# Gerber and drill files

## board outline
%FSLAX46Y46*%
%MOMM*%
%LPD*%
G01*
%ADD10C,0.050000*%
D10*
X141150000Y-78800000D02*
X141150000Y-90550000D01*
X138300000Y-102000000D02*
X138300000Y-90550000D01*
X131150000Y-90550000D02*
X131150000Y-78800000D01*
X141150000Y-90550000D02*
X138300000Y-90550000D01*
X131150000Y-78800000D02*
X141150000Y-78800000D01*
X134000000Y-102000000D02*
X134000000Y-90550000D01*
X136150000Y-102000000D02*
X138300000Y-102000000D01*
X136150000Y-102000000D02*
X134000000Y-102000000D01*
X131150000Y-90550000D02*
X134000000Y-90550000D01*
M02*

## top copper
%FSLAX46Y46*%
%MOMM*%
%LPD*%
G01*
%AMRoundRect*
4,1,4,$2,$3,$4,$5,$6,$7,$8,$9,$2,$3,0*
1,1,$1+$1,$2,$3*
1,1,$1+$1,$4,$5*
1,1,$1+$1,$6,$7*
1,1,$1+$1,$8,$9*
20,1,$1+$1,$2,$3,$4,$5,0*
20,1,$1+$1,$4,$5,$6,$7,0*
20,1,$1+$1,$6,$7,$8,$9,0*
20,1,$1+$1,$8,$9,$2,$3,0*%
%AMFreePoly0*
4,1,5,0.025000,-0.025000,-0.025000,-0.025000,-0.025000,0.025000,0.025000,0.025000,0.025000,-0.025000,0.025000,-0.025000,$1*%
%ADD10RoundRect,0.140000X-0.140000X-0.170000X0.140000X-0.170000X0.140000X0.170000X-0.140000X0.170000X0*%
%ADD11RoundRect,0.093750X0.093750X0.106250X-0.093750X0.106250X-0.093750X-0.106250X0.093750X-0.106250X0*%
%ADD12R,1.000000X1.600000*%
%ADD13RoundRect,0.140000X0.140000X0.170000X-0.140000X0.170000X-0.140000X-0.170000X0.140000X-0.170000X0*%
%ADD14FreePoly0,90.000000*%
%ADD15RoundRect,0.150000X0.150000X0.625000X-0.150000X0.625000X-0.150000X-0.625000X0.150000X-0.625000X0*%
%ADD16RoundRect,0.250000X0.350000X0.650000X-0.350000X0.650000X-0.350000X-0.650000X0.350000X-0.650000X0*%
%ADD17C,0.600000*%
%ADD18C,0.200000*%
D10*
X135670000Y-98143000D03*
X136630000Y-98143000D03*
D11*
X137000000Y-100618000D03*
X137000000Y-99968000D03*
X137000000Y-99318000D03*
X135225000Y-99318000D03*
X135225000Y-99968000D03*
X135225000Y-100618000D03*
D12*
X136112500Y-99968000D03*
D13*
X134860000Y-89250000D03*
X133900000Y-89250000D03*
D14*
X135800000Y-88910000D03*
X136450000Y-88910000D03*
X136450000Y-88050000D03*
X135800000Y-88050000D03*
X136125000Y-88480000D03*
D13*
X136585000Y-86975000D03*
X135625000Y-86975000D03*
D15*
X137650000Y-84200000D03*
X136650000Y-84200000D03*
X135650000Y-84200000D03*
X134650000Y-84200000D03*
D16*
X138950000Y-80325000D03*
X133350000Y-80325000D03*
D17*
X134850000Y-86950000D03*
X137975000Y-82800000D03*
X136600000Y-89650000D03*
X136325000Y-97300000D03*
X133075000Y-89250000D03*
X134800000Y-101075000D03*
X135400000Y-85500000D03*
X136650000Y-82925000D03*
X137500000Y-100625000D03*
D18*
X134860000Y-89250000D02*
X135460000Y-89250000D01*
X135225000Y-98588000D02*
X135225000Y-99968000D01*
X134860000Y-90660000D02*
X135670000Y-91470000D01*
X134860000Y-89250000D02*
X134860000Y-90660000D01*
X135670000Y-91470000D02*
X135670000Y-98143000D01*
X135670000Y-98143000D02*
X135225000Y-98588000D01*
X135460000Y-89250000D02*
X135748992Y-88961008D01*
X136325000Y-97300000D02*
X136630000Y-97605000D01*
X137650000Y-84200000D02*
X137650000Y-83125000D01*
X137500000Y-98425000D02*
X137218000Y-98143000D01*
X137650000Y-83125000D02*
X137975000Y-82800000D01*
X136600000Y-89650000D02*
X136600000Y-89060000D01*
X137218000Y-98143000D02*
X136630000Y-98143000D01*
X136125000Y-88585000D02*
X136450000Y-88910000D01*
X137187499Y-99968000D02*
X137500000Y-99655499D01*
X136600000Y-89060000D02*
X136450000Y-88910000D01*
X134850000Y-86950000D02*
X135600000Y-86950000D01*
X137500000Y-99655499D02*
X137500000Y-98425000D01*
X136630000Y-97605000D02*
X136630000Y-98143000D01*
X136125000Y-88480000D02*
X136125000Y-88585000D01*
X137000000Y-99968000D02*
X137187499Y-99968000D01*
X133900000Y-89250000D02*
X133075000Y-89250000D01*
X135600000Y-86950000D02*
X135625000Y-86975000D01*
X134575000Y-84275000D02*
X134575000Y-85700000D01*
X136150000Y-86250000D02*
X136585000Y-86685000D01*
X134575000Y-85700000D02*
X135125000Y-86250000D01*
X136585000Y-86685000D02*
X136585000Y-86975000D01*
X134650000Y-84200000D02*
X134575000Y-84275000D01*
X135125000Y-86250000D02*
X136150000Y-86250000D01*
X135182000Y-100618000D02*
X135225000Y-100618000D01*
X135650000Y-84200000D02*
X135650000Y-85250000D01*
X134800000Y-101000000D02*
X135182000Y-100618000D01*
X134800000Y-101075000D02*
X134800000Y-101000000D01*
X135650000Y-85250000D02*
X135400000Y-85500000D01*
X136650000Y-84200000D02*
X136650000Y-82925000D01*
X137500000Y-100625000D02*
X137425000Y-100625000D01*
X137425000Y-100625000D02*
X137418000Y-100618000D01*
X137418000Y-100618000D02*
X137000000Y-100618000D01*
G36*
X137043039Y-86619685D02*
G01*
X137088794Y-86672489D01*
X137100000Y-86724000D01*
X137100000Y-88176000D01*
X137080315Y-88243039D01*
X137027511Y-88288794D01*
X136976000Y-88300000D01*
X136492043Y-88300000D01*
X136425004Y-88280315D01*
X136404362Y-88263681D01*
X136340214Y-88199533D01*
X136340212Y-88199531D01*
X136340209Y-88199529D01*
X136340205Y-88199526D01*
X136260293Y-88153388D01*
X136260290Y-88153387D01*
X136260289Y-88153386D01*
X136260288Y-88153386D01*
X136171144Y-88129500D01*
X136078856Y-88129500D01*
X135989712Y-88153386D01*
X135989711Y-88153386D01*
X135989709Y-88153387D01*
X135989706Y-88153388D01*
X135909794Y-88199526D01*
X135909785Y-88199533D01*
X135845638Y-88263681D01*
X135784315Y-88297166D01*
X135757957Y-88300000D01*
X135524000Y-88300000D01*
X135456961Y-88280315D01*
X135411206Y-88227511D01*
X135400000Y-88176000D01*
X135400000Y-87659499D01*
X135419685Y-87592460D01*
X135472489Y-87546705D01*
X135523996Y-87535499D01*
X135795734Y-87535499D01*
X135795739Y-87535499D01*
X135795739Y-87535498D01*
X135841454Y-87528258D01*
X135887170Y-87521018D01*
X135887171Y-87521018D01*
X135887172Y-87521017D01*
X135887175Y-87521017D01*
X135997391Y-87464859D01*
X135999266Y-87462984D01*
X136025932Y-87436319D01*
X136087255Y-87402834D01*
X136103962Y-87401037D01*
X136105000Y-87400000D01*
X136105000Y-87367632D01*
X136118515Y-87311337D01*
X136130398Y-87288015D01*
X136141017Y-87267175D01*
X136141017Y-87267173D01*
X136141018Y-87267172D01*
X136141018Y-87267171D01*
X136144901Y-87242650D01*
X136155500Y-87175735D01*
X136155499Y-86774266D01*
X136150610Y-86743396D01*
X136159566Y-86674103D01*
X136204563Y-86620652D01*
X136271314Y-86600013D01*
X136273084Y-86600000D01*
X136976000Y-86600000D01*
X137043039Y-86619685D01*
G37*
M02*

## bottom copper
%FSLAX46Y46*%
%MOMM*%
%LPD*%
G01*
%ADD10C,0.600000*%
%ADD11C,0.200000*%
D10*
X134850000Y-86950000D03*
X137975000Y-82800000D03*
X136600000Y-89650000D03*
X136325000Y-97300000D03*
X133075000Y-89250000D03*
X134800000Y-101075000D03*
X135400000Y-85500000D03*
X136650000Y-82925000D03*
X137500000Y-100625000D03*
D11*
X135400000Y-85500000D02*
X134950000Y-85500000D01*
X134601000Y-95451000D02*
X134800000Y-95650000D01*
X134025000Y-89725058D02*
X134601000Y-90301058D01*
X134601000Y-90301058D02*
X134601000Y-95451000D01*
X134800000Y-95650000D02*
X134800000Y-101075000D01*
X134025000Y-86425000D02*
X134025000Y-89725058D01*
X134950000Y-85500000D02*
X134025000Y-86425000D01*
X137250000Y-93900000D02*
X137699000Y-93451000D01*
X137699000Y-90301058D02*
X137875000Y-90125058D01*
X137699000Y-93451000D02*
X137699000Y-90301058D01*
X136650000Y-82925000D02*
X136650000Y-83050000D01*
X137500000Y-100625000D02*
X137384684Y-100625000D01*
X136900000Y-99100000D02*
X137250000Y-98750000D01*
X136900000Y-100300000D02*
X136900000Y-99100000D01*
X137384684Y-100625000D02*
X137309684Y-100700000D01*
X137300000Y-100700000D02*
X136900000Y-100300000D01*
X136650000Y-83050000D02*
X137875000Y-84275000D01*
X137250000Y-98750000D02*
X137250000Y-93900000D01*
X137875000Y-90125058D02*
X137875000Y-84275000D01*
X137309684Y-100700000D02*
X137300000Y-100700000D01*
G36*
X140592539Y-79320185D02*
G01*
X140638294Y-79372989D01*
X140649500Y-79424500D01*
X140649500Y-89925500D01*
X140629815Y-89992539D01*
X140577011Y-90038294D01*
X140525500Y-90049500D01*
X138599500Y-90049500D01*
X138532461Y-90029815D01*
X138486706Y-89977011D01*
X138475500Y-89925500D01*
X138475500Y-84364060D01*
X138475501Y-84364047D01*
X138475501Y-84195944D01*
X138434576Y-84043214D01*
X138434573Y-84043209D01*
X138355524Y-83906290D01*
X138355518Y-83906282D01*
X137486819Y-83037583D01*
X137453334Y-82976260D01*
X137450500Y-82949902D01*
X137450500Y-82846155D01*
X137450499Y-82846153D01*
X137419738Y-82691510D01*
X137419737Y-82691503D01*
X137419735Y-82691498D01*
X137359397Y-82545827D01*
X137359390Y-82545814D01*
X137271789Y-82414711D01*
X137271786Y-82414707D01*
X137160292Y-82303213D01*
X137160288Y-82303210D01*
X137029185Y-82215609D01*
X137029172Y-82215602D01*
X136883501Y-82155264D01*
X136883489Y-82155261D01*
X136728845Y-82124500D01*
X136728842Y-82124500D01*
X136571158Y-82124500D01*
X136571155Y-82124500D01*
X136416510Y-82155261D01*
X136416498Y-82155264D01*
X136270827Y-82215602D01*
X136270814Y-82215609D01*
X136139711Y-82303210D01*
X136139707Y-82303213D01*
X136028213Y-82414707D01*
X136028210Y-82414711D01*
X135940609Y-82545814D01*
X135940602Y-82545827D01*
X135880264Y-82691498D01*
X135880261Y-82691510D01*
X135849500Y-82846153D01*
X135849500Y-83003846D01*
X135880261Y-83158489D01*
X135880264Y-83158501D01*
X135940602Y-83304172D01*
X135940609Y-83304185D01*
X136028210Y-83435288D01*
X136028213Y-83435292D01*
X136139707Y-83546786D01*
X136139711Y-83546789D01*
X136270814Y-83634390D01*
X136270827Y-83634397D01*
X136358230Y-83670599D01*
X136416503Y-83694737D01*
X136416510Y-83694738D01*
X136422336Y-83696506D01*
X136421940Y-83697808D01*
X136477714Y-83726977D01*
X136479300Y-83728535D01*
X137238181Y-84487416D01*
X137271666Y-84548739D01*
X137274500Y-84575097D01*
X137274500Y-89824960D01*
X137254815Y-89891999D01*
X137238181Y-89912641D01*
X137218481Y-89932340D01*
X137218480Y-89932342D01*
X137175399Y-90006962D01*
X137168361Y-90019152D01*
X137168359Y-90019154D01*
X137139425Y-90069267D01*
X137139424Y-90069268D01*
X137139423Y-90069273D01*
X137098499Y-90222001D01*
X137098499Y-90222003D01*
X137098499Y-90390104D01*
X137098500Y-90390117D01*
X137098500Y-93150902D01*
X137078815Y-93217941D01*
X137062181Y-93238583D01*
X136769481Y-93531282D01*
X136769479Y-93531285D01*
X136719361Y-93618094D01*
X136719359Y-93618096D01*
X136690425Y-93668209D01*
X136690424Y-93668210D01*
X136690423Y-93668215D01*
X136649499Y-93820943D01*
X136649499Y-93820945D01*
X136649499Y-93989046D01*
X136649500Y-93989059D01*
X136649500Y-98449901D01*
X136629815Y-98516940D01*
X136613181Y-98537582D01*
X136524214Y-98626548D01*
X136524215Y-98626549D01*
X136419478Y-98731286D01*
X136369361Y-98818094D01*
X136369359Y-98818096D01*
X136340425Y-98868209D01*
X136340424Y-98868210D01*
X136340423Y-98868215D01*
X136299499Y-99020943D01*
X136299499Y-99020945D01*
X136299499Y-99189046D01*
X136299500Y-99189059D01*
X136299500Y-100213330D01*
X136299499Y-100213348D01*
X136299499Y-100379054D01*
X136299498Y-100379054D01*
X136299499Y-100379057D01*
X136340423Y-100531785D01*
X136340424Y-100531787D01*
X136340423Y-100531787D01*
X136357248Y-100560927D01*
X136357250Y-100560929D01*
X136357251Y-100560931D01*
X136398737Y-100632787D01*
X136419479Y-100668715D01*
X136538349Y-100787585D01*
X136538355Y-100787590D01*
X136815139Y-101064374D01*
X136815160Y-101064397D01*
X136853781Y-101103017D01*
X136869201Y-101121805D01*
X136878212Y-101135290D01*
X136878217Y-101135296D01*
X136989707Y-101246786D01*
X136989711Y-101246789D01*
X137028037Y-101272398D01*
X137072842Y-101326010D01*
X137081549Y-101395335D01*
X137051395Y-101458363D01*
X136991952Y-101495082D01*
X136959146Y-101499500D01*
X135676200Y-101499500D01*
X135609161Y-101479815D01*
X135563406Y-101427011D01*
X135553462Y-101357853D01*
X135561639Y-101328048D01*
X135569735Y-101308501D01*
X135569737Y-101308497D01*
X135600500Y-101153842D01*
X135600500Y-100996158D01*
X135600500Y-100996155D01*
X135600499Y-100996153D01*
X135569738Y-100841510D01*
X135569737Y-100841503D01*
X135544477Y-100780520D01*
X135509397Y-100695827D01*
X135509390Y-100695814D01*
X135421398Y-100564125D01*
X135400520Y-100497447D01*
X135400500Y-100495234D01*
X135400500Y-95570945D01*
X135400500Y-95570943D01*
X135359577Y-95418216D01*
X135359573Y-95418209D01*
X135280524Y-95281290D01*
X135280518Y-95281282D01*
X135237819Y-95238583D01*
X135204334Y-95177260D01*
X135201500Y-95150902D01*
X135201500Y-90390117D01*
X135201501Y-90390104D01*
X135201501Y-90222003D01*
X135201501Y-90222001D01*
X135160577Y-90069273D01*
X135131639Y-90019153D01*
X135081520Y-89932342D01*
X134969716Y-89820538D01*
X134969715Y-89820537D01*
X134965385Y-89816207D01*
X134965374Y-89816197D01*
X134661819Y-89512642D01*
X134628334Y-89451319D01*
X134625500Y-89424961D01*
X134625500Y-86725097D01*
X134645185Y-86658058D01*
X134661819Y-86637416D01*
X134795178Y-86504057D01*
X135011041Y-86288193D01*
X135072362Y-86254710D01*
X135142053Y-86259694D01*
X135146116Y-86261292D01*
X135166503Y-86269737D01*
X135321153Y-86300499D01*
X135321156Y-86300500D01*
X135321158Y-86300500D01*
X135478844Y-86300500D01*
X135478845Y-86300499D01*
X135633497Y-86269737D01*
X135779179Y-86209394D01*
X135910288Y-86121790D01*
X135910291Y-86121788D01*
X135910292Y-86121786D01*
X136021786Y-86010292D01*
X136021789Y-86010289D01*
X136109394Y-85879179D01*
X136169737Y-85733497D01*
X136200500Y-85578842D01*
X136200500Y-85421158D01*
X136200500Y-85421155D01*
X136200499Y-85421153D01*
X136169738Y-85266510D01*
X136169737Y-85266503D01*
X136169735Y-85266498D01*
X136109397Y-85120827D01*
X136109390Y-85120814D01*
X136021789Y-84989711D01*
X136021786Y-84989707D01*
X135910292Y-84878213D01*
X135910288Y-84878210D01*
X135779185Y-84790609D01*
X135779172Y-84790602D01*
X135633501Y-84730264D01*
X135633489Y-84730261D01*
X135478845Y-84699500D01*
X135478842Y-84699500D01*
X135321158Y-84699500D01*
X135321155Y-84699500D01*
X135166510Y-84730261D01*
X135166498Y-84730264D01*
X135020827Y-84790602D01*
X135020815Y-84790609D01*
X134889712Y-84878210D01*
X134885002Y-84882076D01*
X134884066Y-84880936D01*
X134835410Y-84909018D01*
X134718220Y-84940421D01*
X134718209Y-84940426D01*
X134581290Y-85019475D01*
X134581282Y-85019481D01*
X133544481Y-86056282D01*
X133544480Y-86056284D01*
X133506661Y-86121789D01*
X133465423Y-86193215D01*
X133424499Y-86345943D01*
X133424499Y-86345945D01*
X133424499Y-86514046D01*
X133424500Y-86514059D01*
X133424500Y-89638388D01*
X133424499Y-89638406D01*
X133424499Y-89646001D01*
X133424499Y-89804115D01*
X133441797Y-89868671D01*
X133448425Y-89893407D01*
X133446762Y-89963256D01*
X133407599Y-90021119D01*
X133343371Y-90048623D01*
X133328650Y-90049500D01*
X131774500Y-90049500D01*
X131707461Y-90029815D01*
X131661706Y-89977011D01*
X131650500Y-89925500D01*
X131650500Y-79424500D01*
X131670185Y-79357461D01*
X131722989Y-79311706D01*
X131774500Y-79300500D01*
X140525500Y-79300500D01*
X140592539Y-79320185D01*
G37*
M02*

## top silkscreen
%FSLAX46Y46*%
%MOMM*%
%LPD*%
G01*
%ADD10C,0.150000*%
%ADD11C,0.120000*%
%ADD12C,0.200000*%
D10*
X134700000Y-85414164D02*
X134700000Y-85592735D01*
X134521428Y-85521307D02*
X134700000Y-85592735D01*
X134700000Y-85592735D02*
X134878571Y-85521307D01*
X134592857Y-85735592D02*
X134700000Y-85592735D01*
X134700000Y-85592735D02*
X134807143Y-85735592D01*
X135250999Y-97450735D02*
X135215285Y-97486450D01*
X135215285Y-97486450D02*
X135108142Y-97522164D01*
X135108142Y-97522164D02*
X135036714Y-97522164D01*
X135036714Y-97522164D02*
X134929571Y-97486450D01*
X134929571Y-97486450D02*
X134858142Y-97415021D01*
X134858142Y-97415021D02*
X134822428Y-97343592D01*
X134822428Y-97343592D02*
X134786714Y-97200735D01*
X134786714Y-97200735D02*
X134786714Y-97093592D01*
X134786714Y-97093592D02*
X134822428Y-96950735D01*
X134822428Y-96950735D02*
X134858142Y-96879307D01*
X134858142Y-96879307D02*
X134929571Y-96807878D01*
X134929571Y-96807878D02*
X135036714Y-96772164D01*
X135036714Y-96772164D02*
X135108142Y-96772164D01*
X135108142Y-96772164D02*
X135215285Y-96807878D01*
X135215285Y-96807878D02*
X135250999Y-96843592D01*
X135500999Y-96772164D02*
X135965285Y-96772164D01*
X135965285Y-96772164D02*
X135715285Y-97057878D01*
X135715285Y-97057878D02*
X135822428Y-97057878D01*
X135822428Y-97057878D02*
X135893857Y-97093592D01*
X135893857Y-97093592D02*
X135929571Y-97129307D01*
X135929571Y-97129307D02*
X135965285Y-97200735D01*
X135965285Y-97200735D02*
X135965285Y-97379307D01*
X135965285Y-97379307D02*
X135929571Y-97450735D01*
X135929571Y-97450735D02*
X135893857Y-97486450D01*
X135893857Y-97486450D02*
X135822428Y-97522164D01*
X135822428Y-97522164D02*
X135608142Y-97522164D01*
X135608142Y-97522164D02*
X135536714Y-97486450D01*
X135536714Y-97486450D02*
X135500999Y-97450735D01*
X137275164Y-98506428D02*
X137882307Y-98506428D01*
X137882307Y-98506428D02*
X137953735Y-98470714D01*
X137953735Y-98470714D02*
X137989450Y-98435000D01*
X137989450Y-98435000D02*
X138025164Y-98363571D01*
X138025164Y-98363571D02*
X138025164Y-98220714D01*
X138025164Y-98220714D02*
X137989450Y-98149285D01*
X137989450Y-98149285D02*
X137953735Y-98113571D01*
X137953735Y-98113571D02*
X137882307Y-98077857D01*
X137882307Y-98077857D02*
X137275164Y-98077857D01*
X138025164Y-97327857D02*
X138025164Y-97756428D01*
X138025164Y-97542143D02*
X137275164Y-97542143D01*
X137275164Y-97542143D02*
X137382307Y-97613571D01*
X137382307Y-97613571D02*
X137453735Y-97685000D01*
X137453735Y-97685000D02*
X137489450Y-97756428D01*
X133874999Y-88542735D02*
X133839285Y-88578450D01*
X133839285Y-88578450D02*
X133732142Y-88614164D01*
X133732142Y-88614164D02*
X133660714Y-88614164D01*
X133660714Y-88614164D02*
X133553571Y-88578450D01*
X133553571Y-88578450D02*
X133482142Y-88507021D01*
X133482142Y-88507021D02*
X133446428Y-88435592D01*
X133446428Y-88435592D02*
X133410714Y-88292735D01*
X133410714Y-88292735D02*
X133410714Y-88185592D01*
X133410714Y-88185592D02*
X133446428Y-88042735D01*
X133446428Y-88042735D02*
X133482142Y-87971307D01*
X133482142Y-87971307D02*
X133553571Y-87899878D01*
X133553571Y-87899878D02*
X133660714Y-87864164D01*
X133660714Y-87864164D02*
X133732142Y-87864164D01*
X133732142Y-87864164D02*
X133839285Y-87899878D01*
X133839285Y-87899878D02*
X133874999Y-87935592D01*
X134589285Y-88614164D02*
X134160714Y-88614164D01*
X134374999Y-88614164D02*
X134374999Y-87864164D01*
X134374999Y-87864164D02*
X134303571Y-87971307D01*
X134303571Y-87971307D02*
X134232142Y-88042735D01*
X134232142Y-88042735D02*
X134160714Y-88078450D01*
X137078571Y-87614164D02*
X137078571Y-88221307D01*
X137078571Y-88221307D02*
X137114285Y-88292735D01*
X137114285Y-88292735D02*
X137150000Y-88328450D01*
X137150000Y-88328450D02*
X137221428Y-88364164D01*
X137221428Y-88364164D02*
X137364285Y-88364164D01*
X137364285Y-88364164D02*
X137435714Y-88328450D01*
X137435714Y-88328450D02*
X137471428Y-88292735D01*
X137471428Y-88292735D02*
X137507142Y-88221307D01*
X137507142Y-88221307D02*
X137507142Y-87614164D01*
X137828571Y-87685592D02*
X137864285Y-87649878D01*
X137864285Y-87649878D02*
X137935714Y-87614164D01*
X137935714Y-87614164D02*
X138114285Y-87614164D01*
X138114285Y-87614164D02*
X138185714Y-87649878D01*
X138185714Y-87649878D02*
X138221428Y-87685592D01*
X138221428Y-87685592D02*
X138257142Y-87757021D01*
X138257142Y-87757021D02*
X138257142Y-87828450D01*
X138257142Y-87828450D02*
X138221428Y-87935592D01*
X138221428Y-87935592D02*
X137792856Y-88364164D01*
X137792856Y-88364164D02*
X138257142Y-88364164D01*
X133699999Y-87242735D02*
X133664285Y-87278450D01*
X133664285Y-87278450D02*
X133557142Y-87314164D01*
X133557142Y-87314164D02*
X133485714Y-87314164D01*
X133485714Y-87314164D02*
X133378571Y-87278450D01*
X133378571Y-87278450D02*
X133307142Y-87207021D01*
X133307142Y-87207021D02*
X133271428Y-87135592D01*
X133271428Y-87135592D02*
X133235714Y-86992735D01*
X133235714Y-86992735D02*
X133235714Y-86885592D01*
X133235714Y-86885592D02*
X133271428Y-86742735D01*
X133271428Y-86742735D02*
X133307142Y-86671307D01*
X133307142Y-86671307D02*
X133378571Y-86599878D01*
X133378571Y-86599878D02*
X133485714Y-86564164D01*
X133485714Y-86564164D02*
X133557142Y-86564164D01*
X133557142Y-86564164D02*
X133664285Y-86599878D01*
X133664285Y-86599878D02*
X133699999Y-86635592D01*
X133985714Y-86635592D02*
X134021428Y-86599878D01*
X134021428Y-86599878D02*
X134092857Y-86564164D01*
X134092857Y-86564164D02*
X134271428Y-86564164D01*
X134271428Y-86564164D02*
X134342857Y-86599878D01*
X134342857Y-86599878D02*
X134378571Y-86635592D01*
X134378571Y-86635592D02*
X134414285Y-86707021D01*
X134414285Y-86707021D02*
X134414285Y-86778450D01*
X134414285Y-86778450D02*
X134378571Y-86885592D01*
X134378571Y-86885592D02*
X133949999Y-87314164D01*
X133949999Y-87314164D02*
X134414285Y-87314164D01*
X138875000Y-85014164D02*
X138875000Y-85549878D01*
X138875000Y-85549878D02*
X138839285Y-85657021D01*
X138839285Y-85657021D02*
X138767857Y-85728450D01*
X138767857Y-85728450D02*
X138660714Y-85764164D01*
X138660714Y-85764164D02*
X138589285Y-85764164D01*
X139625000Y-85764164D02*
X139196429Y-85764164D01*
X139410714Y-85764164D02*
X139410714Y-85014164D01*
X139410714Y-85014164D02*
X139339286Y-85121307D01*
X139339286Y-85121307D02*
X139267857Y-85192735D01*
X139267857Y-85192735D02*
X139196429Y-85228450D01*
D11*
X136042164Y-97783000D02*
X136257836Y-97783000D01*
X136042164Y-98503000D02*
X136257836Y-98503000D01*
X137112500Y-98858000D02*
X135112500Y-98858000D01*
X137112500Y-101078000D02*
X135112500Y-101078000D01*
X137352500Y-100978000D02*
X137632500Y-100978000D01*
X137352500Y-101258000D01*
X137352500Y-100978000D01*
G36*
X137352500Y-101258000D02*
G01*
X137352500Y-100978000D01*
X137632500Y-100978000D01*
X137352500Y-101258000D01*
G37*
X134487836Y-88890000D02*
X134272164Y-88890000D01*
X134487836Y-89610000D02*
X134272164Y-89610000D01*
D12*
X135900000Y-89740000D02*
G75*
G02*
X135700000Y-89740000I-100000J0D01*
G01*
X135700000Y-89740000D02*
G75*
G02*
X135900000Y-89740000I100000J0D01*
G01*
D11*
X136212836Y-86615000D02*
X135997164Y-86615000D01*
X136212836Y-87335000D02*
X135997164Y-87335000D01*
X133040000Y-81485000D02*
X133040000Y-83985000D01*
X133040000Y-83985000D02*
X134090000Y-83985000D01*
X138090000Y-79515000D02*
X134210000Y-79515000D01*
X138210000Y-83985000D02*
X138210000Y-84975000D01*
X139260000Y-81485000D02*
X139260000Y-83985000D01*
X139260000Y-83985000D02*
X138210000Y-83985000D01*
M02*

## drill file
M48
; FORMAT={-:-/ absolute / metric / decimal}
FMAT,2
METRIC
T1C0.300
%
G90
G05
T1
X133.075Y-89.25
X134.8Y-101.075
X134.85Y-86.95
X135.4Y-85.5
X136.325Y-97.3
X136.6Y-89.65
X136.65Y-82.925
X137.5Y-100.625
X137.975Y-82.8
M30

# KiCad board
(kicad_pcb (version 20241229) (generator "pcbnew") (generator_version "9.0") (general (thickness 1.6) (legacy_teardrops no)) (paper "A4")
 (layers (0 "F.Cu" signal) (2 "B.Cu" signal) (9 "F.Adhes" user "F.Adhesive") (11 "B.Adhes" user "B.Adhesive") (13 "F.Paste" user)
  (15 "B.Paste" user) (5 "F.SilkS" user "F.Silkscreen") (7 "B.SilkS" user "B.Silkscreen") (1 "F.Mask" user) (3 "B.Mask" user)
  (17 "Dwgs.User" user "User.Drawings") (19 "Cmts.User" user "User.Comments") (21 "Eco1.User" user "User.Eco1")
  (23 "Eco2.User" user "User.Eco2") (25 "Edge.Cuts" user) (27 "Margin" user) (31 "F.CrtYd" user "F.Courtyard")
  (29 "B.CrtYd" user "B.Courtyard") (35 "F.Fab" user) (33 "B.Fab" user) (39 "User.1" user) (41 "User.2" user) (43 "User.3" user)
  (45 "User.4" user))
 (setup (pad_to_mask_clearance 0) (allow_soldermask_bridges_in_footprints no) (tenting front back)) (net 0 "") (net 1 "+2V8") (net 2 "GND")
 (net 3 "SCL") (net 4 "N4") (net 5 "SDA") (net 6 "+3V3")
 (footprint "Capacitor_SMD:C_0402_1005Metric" (layer "F.Cu") (at 136.15 98.143)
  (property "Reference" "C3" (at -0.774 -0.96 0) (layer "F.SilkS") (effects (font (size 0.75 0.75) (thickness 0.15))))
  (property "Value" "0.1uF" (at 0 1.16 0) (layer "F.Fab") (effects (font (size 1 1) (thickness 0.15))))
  (fp_line (start -0.107836 -0.36) (end 0.107836 -0.36) (stroke (width 0.12) (type solid)) (layer "F.SilkS"))
  (fp_line (start -0.107836 0.36) (end 0.107836 0.36) (stroke (width 0.12) (type solid)) (layer "F.SilkS"))
  (pad "1" smd roundrect (at -0.48 0) (size 0.56 0.62) (layers "F.Cu" "F.Mask" "F.Paste") (roundrect_rratio 0.25) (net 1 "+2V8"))
  (pad "2" smd roundrect (at 0.48 0) (size 0.56 0.62) (layers "F.Cu" "F.Mask" "F.Paste") (roundrect_rratio 0.25) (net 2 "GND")))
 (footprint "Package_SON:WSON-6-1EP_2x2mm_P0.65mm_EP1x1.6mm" (layer "F.Cu") (at 136.1125 99.968 180)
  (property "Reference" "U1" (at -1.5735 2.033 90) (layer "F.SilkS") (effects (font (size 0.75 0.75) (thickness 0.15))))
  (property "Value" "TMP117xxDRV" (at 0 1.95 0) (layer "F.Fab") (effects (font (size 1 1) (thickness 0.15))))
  (fp_line (start -1 1.11) (end 1 1.11) (stroke (width 0.12) (type solid)) (layer "F.SilkS"))
  (fp_line (start -1 -1.11) (end 1 -1.11) (stroke (width 0.12) (type solid)) (layer "F.SilkS"))
  (fp_poly (pts (xy -1.24 -1.01) (xy -1.52 -1.01) (xy -1.24 -1.29)) (stroke (width 0.12) (type solid)) (fill yes) (layer "F.SilkS"))
  (pad "" smd roundrect (at 0 -0.4 180) (size 0.81 0.64) (layers "F.Paste") (roundrect_rratio 0.25))
  (pad "" smd roundrect (at 0 0.4 180) (size 0.81 0.64) (layers "F.Paste") (roundrect_rratio 0.25))
  (pad "1" smd roundrect (at -0.8875 -0.65 180) (size 0.375 0.4) (layers "F.Cu" "F.Mask" "F.Paste") (roundrect_rratio 0.25) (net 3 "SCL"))
  (pad "2" smd roundrect (at -0.8875 0 180) (size 0.375 0.4) (layers "F.Cu" "F.Mask" "F.Paste") (roundrect_rratio 0.25) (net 2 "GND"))
  (pad "3" smd roundrect (at -0.8875 0.65 180) (size 0.375 0.4) (layers "F.Cu" "F.Mask" "F.Paste") (roundrect_rratio 0.25) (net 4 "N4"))
  (pad "4" smd roundrect (at 0.8875 0.65 180) (size 0.375 0.4) (layers "F.Cu" "F.Mask" "F.Paste") (roundrect_rratio 0.25) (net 1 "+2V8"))
  (pad "5" smd roundrect (at 0.8875 0 180) (size 0.375 0.4) (layers "F.Cu" "F.Mask" "F.Paste") (roundrect_rratio 0.25) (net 1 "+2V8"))
  (pad "6" smd roundrect (at 0.8875 -0.65 180) (size 0.375 0.4) (layers "F.Cu" "F.Mask" "F.Paste") (roundrect_rratio 0.25) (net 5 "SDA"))
  (pad "7" smd rect (at 0 0 180) (size 1 1.6) (layers "F.Cu" "F.Mask") (zone_connect 2)))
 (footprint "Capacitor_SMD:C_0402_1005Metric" (layer "F.Cu") (at 134.38 89.25 180)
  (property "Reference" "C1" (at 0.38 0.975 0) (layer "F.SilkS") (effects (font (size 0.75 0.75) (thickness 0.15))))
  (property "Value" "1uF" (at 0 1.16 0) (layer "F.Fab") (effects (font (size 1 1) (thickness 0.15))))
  (fp_line (start -0.107836 0.36) (end 0.107836 0.36) (stroke (width 0.12) (type solid)) (layer "F.SilkS"))
  (fp_line (start -0.107836 -0.36) (end 0.107836 -0.36) (stroke (width 0.12) (type solid)) (layer "F.SilkS"))
  (pad "1" smd roundrect (at -0.48 0 180) (size 0.56 0.62) (layers "F.Cu" "F.Mask" "F.Paste") (roundrect_rratio 0.25) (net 1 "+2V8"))
  (pad "2" smd roundrect (at 0.48 0 180) (size 0.56 0.62) (layers "F.Cu" "F.Mask" "F.Paste") (roundrect_rratio 0.25) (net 2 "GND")))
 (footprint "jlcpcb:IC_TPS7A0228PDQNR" (layer "F.Cu") (at 136.125 88.48 90)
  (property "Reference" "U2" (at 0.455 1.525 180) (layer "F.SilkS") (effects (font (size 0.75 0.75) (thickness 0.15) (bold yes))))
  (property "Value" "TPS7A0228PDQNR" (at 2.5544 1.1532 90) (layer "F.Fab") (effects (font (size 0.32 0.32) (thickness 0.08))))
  (fp_circle (center -1.26 -0.325) (end -1.16 -0.325) (stroke (width 0.2) (type solid)) (fill no) (layer "F.SilkS"))
  (pad "1" smd custom (at -0.43 -0.325 90) (size 0.05 0.05) (layers "F.Cu") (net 1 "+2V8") (options (clearance outline) (anchor rect))
   (primitives))
  (pad "2" smd custom (at -0.43 0.325 90) (size 0.05 0.05) (layers "F.Cu") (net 2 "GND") (options (clearance outline) (anchor rect))
   (primitives))
  (pad "3" smd custom (at 0.43 0.325 90) (size 0.05 0.05) (layers "F.Cu") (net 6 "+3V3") (options (clearance outline) (anchor rect))
   (primitives))
  (pad "4" smd custom (at 0.43 -0.325 90) (size 0.05 0.05) (layers "F.Cu") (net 6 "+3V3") (options (clearance outline) (anchor rect))
   (primitives))
  (pad "5" smd custom (at 0 0 90) (size 0.05 0.05) (layers "F.Cu") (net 2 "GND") (options (clearance outline) (anchor rect)) (primitives)))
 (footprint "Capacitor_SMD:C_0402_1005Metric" (layer "F.Cu") (at 136.105 86.975 180)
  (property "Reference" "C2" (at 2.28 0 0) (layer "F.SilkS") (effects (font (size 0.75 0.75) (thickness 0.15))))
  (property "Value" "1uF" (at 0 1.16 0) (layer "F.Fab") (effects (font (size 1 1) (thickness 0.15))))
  (fp_line (start -0.107836 0.36) (end 0.107836 0.36) (stroke (width 0.12) (type solid)) (layer "F.SilkS"))
  (fp_line (start -0.107836 -0.36) (end 0.107836 -0.36) (stroke (width 0.12) (type solid)) (layer "F.SilkS"))
  (pad "1" smd roundrect (at -0.48 0 180) (size 0.56 0.62) (layers "F.Cu" "F.Mask" "F.Paste") (roundrect_rratio 0.25) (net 6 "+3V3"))
  (pad "2" smd roundrect (at 0.48 0 180) (size 0.56 0.62) (layers "F.Cu" "F.Mask" "F.Paste") (roundrect_rratio 0.25) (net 2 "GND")))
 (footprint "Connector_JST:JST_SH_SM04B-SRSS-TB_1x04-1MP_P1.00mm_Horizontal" (layer "F.Cu") (at 136.15 82.2 180)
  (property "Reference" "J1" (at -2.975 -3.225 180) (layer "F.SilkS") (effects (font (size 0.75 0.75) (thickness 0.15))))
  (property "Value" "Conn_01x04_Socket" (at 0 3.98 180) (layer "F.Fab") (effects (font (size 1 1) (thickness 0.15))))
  (fp_line (start 3.11 0.715) (end 3.11 -1.785) (stroke (width 0.12) (type solid)) (layer "F.SilkS"))
  (fp_line (start 3.11 -1.785) (end 2.06 -1.785) (stroke (width 0.12) (type solid)) (layer "F.SilkS"))
  (fp_line (start -1.94 2.685) (end 1.94 2.685) (stroke (width 0.12) (type solid)) (layer "F.SilkS"))
  (fp_line (start -2.06 -1.785) (end -2.06 -2.775) (stroke (width 0.12) (type solid)) (layer "F.SilkS"))
  (fp_line (start -3.11 0.715) (end -3.11 -1.785) (stroke (width 0.12) (type solid)) (layer "F.SilkS"))
  (fp_line (start -3.11 -1.785) (end -2.06 -1.785) (stroke (width 0.12) (type solid)) (layer "F.SilkS"))
  (pad "1" smd roundrect (at -1.5 -2 180) (size 0.6 1.55) (layers "F.Cu" "F.Mask" "F.Paste") (roundrect_rratio 0.25) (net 2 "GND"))
  (pad "2" smd roundrect (at -0.5 -2 180) (size 0.6 1.55) (layers "F.Cu" "F.Mask" "F.Paste") (roundrect_rratio 0.25) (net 3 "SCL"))
  (pad "3" smd roundrect (at 0.5 -2 180) (size 0.6 1.55) (layers "F.Cu" "F.Mask" "F.Paste") (roundrect_rratio 0.25) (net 5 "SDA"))
  (pad "4" smd roundrect (at 1.5 -2 180) (size 0.6 1.55) (layers "F.Cu" "F.Mask" "F.Paste") (roundrect_rratio 0.25) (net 6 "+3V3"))
  (pad "MP" smd roundrect (at -2.8 1.875 180) (size 1.2 1.8) (layers "F.Cu" "F.Mask" "F.Paste") (roundrect_rratio 0.208333))
  (pad "MP" smd roundrect (at 2.8 1.875 180) (size 1.2 1.8) (layers "F.Cu" "F.Mask" "F.Paste") (roundrect_rratio 0.208333)))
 (gr_line (start 141.15 78.8) (end 141.15 90.55) (stroke (width 0.05) (type solid)) (layer "Edge.Cuts"))
 (gr_line (start 138.3 102) (end 138.3 90.55) (stroke (width 0.05) (type default)) (layer "Edge.Cuts"))
 (gr_line (start 131.15 90.55) (end 131.15 78.8) (stroke (width 0.05) (type solid)) (layer "Edge.Cuts"))
 (gr_line (start 141.15 90.55) (end 138.3 90.55) (stroke (width 0.05) (type solid)) (layer "Edge.Cuts"))
 (gr_line (start 131.15 78.8) (end 141.15 78.8) (stroke (width 0.05) (type solid)) (layer "Edge.Cuts"))
 (gr_line (start 134 102) (end 134 90.55) (stroke (width 0.05) (type default)) (layer "Edge.Cuts"))
 (gr_line (start 136.15 102) (end 138.3 102) (stroke (width 0.05) (type solid)) (layer "Edge.Cuts"))
 (gr_line (start 136.15 102) (end 134 102) (stroke (width 0.05) (type solid)) (layer "Edge.Cuts"))
 (gr_line (start 131.15 90.55) (end 134 90.55) (stroke (width 0.05) (type solid)) (layer "Edge.Cuts"))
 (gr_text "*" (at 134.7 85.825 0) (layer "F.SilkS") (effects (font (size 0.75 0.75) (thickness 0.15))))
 (segment (start 134.86 89.25) (end 135.46 89.25) (width 0.2) (layer "F.Cu") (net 1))
 (segment (start 135.225 98.588) (end 135.225 99.968) (width 0.2) (layer "F.Cu") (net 1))
 (segment (start 134.86 90.66) (end 135.67 91.47) (width 0.2) (layer "F.Cu") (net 1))
 (segment (start 134.86 89.25) (end 134.86 90.66) (width 0.2) (layer "F.Cu") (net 1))
 (segment (start 135.67 91.47) (end 135.67 98.143) (width 0.2) (layer "F.Cu") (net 1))
 (segment (start 135.67 98.143) (end 135.225 98.588) (width 0.2) (layer "F.Cu") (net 1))
 (segment (start 135.46 89.25) (end 135.748992 88.961008) (width 0.2) (layer "F.Cu") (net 1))
 (segment (start 136.325 97.3) (end 136.63 97.605) (width 0.2) (layer "F.Cu") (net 2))
 (segment (start 137.65 84.2) (end 137.65 83.125) (width 0.2) (layer "F.Cu") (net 2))
 (segment (start 137.5 98.425) (end 137.218 98.143) (width 0.2) (layer "F.Cu") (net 2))
 (segment (start 137.65 83.125) (end 137.975 82.8) (width 0.2) (layer "F.Cu") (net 2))
 (segment (start 136.6 89.65) (end 136.6 89.06) (width 0.2) (layer "F.Cu") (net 2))
 (segment (start 137.218 98.143) (end 136.63 98.143) (width 0.2) (layer "F.Cu") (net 2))
 (segment (start 136.125 88.585) (end 136.45 88.91) (width 0.2) (layer "F.Cu") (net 2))
 (segment (start 137.187499 99.968) (end 137.5 99.655499) (width 0.2) (layer "F.Cu") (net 2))
 (segment (start 136.6 89.06) (end 136.45 88.91) (width 0.2) (layer "F.Cu") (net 2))
 (segment (start 134.85 86.95) (end 135.6 86.95) (width 0.2) (layer "F.Cu") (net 2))
 (segment (start 137.5 99.655499) (end 137.5 98.425) (width 0.2) (layer "F.Cu") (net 2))
 (segment (start 136.63 97.605) (end 136.63 98.143) (width 0.2) (layer "F.Cu") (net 2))
 (segment (start 136.125 88.48) (end 136.125 88.585) (width 0.2) (layer "F.Cu") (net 2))
 (segment (start 137 99.968) (end 137.187499 99.968) (width 0.2) (layer "F.Cu") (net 2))
 (segment (start 133.9 89.25) (end 133.075 89.25) (width 0.2) (layer "F.Cu") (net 2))
 (segment (start 135.6 86.95) (end 135.625 86.975) (width 0.2) (layer "F.Cu") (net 2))
 (via (at 134.85 86.95) (size 0.6) (drill 0.3) (layers "F.Cu" "B.Cu") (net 2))
 (via (at 137.975 82.8) (size 0.6) (drill 0.3) (layers "F.Cu" "B.Cu") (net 2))
 (via (at 136.6 89.65) (size 0.6) (drill 0.3) (layers "F.Cu" "B.Cu") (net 2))
 (via (at 136.325 97.3) (size 0.6) (drill 0.3) (layers "F.Cu" "B.Cu") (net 2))
 (via (at 133.075 89.25) (size 0.6) (drill 0.3) (layers "F.Cu" "B.Cu") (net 2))
 (segment (start 134.575 84.275) (end 134.575 85.7) (width 0.2) (layer "F.Cu") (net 6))
 (segment (start 136.15 86.25) (end 136.585 86.685) (width 0.2) (layer "F.Cu") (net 6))
 (segment (start 134.575 85.7) (end 135.125 86.25) (width 0.2) (layer "F.Cu") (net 6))
 (segment (start 136.585 86.685) (end 136.585 86.975) (width 0.2) (layer "F.Cu") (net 6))
 (segment (start 134.65 84.2) (end 134.575 84.275) (width 0.2) (layer "F.Cu") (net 6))
 (segment (start 135.125 86.25) (end 136.15 86.25) (width 0.2) (layer "F.Cu") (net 6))
 (segment (start 135.182 100.618) (end 135.225 100.618) (width 0.2) (layer "F.Cu") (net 5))
 (segment (start 135.65 84.2) (end 135.65 85.25) (width 0.2) (layer "F.Cu") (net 5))
 (segment (start 134.8 101) (end 135.182 100.618) (width 0.2) (layer "F.Cu") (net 5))
 (segment (start 134.8 101.075) (end 134.8 101) (width 0.2) (layer "F.Cu") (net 5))
 (segment (start 135.65 85.25) (end 135.4 85.5) (width 0.2) (layer "F.Cu") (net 5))
 (via (at 134.8 101.075) (size 0.6) (drill 0.3) (layers "F.Cu" "B.Cu") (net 5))
 (via (at 135.4 85.5) (size 0.6) (drill 0.3) (layers "F.Cu" "B.Cu") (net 5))
 (segment (start 135.4 85.5) (end 134.95 85.5) (width 0.2) (layer "B.Cu") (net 5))
 (segment (start 134.601 95.451) (end 134.8 95.65) (width 0.2) (layer "B.Cu") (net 5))
 (segment (start 134.025 89.725058) (end 134.601 90.301058) (width 0.2) (layer "B.Cu") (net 5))
 (segment (start 134.601 90.301058) (end 134.601 95.451) (width 0.2) (layer "B.Cu") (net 5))
 (segment (start 134.8 95.65) (end 134.8 101.075) (width 0.2) (layer "B.Cu") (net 5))
 (segment (start 134.025 86.425) (end 134.025 89.725058) (width 0.2) (layer "B.Cu") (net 5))
 (segment (start 134.95 85.5) (end 134.025 86.425) (width 0.2) (layer "B.Cu") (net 5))
 (segment (start 136.65 84.2) (end 136.65 82.925) (width 0.2) (layer "F.Cu") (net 3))
 (segment (start 137.5 100.625) (end 137.425 100.625) (width 0.2) (layer "F.Cu") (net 3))
 (segment (start 137.425 100.625) (end 137.418 100.618) (width 0.2) (layer "F.Cu") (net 3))
 (segment (start 137.418 100.618) (end 137 100.618) (width 0.2) (layer "F.Cu") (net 3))
 (via (at 136.65 82.925) (size 0.6) (drill 0.3) (layers "F.Cu" "B.Cu") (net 3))
 (via (at 137.5 100.625) (size 0.6) (drill 0.3) (layers "F.Cu" "B.Cu") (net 3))
 (segment (start 137.25 93.9) (end 137.699 93.451) (width 0.2) (layer "B.Cu") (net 3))
 (segment (start 137.699 90.301058) (end 137.875 90.125058) (width 0.2) (layer "B.Cu") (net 3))
 (segment (start 137.699 93.451) (end 137.699 90.301058) (width 0.2) (layer "B.Cu") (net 3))
 (segment (start 136.65 82.925) (end 136.65 83.05) (width 0.2) (layer "B.Cu") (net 3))
 (segment (start 137.5 100.625) (end 137.384684 100.625) (width 0.2) (layer "B.Cu") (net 3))
 (segment (start 136.9 99.1) (end 137.25 98.75) (width 0.2) (layer "B.Cu") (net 3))
 (segment (start 136.9 100.3) (end 136.9 99.1) (width 0.2) (layer "B.Cu") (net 3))
 (segment (start 137.384684 100.625) (end 137.309684 100.7) (width 0.2) (layer "B.Cu") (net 3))
 (segment (start 137.3 100.7) (end 136.9 100.3) (width 0.2) (layer "B.Cu") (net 3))
 (segment (start 136.65 83.05) (end 137.875 84.275) (width 0.2) (layer "B.Cu") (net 3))
 (segment (start 137.25 98.75) (end 137.25 93.9) (width 0.2) (layer "B.Cu") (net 3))
 (segment (start 137.875 90.125058) (end 137.875 84.275) (width 0.2) (layer "B.Cu") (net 3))
 (segment (start 137.309684 100.7) (end 137.3 100.7) (width 0.2) (layer "B.Cu") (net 3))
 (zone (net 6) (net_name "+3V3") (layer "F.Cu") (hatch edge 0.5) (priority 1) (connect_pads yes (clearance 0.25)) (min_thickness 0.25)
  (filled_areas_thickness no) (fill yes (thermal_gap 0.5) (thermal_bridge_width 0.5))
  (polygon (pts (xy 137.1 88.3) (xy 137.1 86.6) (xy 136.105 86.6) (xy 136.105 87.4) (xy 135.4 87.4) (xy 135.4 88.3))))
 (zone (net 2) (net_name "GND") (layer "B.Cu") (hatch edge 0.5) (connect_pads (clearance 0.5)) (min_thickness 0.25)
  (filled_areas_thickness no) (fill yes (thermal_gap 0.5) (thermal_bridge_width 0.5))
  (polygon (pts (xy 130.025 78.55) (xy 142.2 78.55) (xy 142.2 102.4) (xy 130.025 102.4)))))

